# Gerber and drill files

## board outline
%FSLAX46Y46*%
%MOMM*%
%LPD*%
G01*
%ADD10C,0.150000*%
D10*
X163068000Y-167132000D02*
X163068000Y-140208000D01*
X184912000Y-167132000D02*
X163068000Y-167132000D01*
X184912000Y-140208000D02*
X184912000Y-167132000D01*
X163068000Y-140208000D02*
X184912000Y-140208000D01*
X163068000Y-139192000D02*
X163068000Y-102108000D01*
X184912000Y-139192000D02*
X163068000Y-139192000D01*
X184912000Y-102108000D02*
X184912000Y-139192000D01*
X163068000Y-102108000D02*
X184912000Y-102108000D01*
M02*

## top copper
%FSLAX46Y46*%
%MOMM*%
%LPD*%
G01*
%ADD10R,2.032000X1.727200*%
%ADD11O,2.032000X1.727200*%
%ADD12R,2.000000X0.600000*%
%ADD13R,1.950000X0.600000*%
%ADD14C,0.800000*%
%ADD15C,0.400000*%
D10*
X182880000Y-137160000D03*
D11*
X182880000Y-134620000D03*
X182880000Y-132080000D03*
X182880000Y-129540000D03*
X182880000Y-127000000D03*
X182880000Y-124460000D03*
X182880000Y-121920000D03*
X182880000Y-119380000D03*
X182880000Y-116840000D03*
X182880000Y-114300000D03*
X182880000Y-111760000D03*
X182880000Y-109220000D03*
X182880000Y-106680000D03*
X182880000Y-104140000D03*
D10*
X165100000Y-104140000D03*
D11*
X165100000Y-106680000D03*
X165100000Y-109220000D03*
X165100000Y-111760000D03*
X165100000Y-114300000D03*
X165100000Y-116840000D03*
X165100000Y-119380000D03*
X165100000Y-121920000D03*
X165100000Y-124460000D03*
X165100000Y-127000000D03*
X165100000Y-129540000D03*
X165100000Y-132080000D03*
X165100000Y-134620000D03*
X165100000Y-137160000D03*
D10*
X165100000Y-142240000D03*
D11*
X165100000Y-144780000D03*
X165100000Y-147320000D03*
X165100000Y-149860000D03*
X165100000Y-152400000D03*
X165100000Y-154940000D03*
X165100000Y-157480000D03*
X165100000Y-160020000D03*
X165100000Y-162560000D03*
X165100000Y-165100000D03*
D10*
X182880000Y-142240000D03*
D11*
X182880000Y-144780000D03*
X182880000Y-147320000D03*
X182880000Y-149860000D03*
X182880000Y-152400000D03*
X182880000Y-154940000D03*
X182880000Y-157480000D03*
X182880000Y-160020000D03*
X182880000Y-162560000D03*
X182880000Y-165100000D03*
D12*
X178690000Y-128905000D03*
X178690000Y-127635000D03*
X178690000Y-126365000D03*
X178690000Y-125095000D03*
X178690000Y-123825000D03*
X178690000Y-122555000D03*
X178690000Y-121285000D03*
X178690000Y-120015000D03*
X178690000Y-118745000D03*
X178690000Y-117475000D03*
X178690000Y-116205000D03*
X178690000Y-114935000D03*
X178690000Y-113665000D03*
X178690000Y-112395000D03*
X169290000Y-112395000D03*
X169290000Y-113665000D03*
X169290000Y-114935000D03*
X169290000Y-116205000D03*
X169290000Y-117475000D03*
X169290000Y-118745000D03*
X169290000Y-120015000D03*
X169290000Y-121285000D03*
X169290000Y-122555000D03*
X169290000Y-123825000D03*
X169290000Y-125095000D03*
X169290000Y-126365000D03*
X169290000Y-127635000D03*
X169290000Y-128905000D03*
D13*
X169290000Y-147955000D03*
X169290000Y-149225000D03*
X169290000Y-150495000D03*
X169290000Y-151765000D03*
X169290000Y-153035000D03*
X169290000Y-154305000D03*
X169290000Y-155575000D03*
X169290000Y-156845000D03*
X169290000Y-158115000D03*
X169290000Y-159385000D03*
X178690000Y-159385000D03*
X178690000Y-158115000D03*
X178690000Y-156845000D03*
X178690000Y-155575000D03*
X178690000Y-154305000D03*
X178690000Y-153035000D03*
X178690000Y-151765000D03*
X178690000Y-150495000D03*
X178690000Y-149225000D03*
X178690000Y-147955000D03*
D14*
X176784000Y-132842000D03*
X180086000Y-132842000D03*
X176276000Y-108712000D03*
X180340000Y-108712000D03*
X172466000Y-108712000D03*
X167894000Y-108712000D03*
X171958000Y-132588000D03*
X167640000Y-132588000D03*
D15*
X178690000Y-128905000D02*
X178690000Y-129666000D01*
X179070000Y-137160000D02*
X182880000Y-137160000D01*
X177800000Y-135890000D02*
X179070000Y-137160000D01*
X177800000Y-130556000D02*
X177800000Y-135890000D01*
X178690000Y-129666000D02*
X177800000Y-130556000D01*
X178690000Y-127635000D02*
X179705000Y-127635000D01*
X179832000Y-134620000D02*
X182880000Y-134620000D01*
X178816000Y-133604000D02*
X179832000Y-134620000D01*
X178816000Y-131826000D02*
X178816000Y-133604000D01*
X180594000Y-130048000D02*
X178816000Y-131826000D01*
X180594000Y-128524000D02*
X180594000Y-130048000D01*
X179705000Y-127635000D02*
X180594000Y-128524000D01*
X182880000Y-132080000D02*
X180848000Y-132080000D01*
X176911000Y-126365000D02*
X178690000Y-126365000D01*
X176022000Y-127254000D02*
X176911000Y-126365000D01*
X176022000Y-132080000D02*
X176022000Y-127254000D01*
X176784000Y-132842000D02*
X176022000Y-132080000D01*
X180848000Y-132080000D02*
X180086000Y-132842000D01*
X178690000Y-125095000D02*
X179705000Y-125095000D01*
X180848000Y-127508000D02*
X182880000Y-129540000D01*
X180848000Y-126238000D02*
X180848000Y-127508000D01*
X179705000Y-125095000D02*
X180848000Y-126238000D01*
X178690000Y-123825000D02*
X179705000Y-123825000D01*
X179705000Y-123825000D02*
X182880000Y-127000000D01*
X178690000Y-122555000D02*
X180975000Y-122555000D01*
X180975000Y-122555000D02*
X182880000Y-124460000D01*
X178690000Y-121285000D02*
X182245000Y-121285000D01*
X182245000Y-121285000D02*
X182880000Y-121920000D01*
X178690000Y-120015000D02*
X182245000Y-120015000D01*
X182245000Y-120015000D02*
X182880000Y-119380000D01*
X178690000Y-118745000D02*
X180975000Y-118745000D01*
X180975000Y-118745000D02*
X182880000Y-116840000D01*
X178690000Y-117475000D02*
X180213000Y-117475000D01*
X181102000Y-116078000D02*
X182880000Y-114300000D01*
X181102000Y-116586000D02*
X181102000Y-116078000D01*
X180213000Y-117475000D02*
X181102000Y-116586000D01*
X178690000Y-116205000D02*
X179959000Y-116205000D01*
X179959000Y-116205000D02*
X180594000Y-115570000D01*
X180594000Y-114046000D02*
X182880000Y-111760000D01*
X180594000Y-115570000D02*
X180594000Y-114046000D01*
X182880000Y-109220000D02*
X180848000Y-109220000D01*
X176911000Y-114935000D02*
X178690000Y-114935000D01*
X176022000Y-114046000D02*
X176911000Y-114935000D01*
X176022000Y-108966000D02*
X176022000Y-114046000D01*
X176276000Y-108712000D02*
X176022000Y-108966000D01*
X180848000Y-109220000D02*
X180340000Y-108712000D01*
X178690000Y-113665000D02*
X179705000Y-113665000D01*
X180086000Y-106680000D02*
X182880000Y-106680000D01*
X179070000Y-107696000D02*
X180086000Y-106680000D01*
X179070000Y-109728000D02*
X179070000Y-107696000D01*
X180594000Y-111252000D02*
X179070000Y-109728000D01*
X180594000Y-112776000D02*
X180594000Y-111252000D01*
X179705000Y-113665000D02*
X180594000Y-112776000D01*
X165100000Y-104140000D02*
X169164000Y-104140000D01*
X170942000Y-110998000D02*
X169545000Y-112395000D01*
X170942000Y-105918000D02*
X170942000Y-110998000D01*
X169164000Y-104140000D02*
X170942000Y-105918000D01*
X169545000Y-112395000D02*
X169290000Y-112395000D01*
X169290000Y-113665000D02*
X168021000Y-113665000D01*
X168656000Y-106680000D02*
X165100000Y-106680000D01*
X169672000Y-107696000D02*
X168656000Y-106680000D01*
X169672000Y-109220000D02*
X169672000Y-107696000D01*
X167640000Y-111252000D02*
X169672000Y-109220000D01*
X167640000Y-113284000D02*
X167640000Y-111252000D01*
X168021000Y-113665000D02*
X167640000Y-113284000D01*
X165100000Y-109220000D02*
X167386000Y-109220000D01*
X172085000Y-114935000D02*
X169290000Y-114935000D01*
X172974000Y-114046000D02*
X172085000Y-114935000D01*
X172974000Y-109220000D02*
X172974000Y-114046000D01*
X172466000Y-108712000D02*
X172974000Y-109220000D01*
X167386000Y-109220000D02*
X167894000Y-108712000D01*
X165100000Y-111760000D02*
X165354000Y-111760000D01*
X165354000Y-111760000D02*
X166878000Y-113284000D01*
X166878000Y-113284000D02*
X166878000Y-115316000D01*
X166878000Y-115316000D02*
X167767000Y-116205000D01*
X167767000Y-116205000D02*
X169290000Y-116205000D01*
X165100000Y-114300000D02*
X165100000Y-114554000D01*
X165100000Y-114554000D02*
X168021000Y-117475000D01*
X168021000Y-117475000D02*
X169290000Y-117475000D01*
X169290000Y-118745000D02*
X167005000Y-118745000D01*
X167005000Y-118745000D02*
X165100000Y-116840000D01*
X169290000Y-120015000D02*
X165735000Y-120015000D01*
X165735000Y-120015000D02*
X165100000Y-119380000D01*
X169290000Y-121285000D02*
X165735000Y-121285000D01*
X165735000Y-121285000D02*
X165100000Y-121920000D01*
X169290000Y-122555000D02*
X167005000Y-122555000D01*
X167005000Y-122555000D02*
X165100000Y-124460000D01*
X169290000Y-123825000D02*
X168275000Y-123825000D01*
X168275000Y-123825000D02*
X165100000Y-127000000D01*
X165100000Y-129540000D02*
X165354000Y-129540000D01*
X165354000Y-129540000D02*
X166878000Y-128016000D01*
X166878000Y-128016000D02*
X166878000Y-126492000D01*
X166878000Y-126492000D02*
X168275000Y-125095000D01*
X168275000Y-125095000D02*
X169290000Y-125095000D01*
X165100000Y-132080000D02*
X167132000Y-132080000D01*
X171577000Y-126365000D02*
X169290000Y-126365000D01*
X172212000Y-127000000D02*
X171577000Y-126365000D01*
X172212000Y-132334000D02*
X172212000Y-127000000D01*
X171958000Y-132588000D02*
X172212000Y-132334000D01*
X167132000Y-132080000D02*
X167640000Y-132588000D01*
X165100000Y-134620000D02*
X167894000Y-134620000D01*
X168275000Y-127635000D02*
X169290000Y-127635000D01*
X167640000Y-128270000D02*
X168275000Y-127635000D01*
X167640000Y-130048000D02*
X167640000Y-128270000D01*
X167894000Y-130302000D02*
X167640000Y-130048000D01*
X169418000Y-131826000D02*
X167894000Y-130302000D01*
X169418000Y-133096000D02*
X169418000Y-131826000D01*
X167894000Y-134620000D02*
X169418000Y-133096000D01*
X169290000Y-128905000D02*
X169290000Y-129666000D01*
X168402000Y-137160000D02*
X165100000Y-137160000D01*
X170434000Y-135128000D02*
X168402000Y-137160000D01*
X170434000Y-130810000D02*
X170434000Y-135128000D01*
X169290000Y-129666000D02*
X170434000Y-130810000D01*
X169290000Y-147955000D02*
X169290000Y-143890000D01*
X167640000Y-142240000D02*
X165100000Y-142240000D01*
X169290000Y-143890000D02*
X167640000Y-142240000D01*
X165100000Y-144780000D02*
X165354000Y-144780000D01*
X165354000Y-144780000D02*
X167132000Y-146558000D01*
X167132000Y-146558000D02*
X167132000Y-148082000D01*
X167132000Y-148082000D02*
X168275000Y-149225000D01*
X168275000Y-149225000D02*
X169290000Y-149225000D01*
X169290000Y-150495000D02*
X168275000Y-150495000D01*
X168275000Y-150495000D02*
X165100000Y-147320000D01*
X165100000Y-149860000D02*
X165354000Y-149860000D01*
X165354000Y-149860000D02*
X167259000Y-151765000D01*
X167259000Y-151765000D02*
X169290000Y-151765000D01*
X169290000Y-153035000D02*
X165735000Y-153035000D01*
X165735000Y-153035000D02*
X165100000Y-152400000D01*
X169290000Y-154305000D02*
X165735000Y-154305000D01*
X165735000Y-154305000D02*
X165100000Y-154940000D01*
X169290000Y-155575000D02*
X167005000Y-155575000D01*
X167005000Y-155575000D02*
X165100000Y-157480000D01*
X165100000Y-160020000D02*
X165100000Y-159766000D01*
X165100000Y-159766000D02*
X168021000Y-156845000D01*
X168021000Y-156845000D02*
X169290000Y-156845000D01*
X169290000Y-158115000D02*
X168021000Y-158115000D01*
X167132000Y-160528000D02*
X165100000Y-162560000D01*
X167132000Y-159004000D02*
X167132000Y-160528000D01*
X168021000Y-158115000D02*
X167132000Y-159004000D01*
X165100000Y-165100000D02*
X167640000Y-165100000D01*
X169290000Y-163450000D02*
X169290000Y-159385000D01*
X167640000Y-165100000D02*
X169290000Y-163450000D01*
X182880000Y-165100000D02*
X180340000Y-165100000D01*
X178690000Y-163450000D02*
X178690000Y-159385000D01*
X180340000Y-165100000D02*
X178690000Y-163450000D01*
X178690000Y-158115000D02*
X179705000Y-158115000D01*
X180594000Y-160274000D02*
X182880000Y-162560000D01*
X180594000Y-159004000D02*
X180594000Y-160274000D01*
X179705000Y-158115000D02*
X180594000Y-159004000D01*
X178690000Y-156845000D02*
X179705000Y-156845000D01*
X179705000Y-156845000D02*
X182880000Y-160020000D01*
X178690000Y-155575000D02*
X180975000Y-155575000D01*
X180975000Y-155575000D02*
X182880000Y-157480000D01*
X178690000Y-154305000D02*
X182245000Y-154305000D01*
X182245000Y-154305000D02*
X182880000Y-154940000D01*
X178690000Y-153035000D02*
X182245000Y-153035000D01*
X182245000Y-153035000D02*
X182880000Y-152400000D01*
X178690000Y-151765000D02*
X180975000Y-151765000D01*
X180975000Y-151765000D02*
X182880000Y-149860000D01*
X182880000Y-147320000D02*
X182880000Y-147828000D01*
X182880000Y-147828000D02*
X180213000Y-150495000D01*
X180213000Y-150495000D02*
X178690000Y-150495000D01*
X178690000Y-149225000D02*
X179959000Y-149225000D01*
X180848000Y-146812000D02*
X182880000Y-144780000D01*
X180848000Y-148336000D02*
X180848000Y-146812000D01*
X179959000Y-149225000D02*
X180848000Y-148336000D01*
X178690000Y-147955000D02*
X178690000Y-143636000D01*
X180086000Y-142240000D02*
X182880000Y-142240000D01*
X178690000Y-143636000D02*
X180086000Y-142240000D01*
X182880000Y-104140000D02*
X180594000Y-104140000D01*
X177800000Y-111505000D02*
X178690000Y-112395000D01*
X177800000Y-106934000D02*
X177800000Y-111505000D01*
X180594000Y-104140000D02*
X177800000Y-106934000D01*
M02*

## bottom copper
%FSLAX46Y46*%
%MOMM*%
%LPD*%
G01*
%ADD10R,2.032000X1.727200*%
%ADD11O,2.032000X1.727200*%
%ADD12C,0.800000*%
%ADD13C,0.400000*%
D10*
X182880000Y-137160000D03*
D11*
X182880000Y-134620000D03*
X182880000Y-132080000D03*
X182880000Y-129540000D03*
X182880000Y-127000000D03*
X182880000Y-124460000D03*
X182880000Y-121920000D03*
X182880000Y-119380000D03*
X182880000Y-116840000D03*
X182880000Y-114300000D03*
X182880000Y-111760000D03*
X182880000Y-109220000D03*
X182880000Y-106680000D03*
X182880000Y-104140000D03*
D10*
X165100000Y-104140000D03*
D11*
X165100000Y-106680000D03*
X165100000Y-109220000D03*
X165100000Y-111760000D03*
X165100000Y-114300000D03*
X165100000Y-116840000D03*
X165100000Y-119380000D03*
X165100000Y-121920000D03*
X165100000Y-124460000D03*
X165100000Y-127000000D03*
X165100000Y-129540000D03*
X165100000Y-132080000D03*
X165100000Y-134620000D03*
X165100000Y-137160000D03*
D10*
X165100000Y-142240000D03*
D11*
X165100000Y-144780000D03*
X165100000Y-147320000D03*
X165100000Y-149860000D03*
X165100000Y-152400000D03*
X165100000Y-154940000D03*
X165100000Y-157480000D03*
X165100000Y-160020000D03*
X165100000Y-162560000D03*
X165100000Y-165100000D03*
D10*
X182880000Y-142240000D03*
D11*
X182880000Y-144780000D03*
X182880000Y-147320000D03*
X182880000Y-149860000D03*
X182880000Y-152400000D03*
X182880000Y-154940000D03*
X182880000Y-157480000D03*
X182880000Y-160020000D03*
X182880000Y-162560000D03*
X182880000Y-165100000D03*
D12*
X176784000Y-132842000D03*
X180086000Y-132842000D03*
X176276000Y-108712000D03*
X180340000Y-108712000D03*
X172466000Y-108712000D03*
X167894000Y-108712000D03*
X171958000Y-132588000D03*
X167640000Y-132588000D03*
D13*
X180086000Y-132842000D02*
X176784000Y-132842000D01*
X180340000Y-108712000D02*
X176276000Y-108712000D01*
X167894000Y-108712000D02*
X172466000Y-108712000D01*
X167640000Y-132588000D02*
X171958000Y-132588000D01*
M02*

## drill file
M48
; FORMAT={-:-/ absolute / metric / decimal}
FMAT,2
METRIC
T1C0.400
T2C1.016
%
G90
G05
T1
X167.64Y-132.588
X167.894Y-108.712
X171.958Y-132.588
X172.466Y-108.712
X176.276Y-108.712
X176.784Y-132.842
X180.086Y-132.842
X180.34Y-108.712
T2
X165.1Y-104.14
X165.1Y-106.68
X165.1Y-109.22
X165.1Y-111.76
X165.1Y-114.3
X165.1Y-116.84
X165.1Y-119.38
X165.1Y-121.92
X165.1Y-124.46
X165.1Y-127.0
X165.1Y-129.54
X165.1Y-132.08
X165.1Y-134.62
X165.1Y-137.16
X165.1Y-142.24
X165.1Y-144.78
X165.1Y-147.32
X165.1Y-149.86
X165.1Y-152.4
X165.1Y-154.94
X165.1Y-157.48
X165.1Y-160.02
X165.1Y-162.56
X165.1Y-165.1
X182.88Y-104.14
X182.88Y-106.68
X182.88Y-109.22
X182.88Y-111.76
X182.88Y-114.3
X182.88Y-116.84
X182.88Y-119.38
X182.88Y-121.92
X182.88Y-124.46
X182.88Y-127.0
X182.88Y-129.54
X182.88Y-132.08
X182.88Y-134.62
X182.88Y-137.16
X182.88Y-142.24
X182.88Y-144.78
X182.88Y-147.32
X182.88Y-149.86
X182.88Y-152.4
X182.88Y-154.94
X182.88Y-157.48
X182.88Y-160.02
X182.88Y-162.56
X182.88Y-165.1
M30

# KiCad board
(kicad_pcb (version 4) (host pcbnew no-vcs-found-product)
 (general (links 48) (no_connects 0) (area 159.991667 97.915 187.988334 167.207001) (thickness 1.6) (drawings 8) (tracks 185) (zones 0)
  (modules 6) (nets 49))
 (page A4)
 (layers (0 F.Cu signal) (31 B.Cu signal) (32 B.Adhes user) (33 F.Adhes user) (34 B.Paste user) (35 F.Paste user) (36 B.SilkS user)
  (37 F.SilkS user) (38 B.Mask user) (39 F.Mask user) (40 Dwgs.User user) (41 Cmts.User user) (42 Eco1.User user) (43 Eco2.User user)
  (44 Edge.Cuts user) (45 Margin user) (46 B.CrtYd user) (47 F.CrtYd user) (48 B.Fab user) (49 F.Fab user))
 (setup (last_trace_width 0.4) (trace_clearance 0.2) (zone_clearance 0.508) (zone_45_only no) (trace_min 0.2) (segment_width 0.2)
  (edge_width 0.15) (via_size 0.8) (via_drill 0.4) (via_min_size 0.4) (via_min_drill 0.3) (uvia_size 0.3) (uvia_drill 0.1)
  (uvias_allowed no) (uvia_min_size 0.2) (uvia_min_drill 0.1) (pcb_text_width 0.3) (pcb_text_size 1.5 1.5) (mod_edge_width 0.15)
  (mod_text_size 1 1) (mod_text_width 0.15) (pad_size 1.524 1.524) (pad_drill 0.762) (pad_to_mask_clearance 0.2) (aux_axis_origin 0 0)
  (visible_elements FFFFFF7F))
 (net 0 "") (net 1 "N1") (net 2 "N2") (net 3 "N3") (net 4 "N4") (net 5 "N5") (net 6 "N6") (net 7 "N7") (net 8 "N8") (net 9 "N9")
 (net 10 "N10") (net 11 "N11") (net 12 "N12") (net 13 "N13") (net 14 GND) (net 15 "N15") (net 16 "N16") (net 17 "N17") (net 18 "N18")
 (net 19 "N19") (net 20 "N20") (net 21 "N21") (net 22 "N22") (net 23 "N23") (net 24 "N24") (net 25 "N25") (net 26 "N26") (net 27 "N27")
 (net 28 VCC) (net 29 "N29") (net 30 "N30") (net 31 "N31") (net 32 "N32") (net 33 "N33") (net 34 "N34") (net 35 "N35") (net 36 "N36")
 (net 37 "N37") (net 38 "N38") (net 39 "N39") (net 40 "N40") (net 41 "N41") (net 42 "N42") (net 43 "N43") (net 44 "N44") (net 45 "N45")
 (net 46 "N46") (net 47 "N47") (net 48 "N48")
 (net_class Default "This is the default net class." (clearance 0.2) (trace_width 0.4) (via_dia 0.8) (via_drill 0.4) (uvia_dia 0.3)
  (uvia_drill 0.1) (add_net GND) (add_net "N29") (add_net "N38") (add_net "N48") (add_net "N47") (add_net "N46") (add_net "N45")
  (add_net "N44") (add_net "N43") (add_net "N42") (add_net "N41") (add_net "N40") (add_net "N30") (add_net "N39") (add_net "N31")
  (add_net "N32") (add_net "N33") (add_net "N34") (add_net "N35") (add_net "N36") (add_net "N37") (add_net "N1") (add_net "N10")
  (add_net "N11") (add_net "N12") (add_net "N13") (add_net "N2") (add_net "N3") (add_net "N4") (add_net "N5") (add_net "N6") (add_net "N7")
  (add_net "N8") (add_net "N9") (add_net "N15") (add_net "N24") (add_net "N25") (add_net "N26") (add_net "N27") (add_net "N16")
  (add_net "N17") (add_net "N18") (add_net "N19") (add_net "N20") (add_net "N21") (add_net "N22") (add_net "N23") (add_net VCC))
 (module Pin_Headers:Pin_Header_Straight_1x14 (layer F.Cu) (at 182.88 137.16 180)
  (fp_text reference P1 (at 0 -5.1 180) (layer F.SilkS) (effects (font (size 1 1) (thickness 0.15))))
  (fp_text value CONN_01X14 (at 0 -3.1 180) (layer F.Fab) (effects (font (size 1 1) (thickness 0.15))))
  (pad 1 thru_hole rect (at 0 0 180) (size 2.032 1.7272) (drill 1.016) (layers *.Cu *.Mask F.SilkS) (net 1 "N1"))
  (pad 2 thru_hole oval (at 0 2.54 180) (size 2.032 1.7272) (drill 1.016) (layers *.Cu *.Mask F.SilkS) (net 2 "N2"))
  (pad 3 thru_hole oval (at 0 5.08 180) (size 2.032 1.7272) (drill 1.016) (layers *.Cu *.Mask F.SilkS) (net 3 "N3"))
  (pad 4 thru_hole oval (at 0 7.62 180) (size 2.032 1.7272) (drill 1.016) (layers *.Cu *.Mask F.SilkS) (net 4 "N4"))
  (pad 5 thru_hole oval (at 0 10.16 180) (size 2.032 1.7272) (drill 1.016) (layers *.Cu *.Mask F.SilkS) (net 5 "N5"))
  (pad 6 thru_hole oval (at 0 12.7 180) (size 2.032 1.7272) (drill 1.016) (layers *.Cu *.Mask F.SilkS) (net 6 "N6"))
  (pad 7 thru_hole oval (at 0 15.24 180) (size 2.032 1.7272) (drill 1.016) (layers *.Cu *.Mask F.SilkS) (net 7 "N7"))
  (pad 8 thru_hole oval (at 0 17.78 180) (size 2.032 1.7272) (drill 1.016) (layers *.Cu *.Mask F.SilkS) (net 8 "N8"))
  (pad 9 thru_hole oval (at 0 20.32 180) (size 2.032 1.7272) (drill 1.016) (layers *.Cu *.Mask F.SilkS) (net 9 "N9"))
  (pad 10 thru_hole oval (at 0 22.86 180) (size 2.032 1.7272) (drill 1.016) (layers *.Cu *.Mask F.SilkS) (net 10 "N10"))
  (pad 11 thru_hole oval (at 0 25.4 180) (size 2.032 1.7272) (drill 1.016) (layers *.Cu *.Mask F.SilkS) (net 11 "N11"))
  (pad 12 thru_hole oval (at 0 27.94 180) (size 2.032 1.7272) (drill 1.016) (layers *.Cu *.Mask F.SilkS) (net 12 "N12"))
  (pad 13 thru_hole oval (at 0 30.48 180) (size 2.032 1.7272) (drill 1.016) (layers *.Cu *.Mask F.SilkS) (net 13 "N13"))
  (pad 14 thru_hole oval (at 0 33.02 180) (size 2.032 1.7272) (drill 1.016) (layers *.Cu *.Mask F.SilkS) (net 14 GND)))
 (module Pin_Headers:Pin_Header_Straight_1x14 (layer F.Cu) (at 165.1 104.14)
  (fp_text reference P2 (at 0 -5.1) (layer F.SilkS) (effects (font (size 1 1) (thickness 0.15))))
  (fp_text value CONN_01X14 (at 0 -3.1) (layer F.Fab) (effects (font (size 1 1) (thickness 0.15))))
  (pad 1 thru_hole rect (at 0 0) (size 2.032 1.7272) (drill 1.016) (layers *.Cu *.Mask F.SilkS) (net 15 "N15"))
  (pad 2 thru_hole oval (at 0 2.54) (size 2.032 1.7272) (drill 1.016) (layers *.Cu *.Mask F.SilkS) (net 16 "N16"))
  (pad 3 thru_hole oval (at 0 5.08) (size 2.032 1.7272) (drill 1.016) (layers *.Cu *.Mask F.SilkS) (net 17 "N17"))
  (pad 4 thru_hole oval (at 0 7.62) (size 2.032 1.7272) (drill 1.016) (layers *.Cu *.Mask F.SilkS) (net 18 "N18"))
  (pad 5 thru_hole oval (at 0 10.16) (size 2.032 1.7272) (drill 1.016) (layers *.Cu *.Mask F.SilkS) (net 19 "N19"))
  (pad 6 thru_hole oval (at 0 12.7) (size 2.032 1.7272) (drill 1.016) (layers *.Cu *.Mask F.SilkS) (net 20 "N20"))
  (pad 7 thru_hole oval (at 0 15.24) (size 2.032 1.7272) (drill 1.016) (layers *.Cu *.Mask F.SilkS) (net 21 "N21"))
  (pad 8 thru_hole oval (at 0 17.78) (size 2.032 1.7272) (drill 1.016) (layers *.Cu *.Mask F.SilkS) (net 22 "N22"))
  (pad 9 thru_hole oval (at 0 20.32) (size 2.032 1.7272) (drill 1.016) (layers *.Cu *.Mask F.SilkS) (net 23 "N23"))
  (pad 10 thru_hole oval (at 0 22.86) (size 2.032 1.7272) (drill 1.016) (layers *.Cu *.Mask F.SilkS) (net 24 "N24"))
  (pad 11 thru_hole oval (at 0 25.4) (size 2.032 1.7272) (drill 1.016) (layers *.Cu *.Mask F.SilkS) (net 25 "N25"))
  (pad 12 thru_hole oval (at 0 27.94) (size 2.032 1.7272) (drill 1.016) (layers *.Cu *.Mask F.SilkS) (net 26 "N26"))
  (pad 13 thru_hole oval (at 0 30.48) (size 2.032 1.7272) (drill 1.016) (layers *.Cu *.Mask F.SilkS) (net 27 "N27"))
  (pad 14 thru_hole oval (at 0 33.02) (size 2.032 1.7272) (drill 1.016) (layers *.Cu *.Mask F.SilkS) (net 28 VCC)))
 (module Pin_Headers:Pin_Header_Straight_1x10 (layer F.Cu) (at 165.1 142.24)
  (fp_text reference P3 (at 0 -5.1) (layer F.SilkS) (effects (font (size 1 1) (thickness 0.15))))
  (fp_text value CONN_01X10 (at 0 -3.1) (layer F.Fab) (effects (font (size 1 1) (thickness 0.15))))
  (pad 1 thru_hole rect (at 0 0) (size 2.032 1.7272) (drill 1.016) (layers *.Cu *.Mask F.SilkS) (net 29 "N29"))
  (pad 2 thru_hole oval (at 0 2.54) (size 2.032 1.7272) (drill 1.016) (layers *.Cu *.Mask F.SilkS) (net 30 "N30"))
  (pad 3 thru_hole oval (at 0 5.08) (size 2.032 1.7272) (drill 1.016) (layers *.Cu *.Mask F.SilkS) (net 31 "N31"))
  (pad 4 thru_hole oval (at 0 7.62) (size 2.032 1.7272) (drill 1.016) (layers *.Cu *.Mask F.SilkS) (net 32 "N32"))
  (pad 5 thru_hole oval (at 0 10.16) (size 2.032 1.7272) (drill 1.016) (layers *.Cu *.Mask F.SilkS) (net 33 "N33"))
  (pad 6 thru_hole oval (at 0 12.7) (size 2.032 1.7272) (drill 1.016) (layers *.Cu *.Mask F.SilkS) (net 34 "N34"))
  (pad 7 thru_hole oval (at 0 15.24) (size 2.032 1.7272) (drill 1.016) (layers *.Cu *.Mask F.SilkS) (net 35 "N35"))
  (pad 8 thru_hole oval (at 0 17.78) (size 2.032 1.7272) (drill 1.016) (layers *.Cu *.Mask F.SilkS) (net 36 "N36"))
  (pad 9 thru_hole oval (at 0 20.32) (size 2.032 1.7272) (drill 1.016) (layers *.Cu *.Mask F.SilkS) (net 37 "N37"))
  (pad 10 thru_hole oval (at 0 22.86) (size 2.032 1.7272) (drill 1.016) (layers *.Cu *.Mask F.SilkS) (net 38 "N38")))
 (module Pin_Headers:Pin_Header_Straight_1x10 (layer F.Cu) (at 182.88 142.24)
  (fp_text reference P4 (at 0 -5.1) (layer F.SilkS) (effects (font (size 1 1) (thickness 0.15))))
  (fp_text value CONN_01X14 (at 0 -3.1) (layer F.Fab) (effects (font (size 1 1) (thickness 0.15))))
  (pad 1 thru_hole rect (at 0 0) (size 2.032 1.7272) (drill 1.016) (layers *.Cu *.Mask F.SilkS) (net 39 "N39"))
  (pad 2 thru_hole oval (at 0 2.54) (size 2.032 1.7272) (drill 1.016) (layers *.Cu *.Mask F.SilkS) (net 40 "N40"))
  (pad 3 thru_hole oval (at 0 5.08) (size 2.032 1.7272) (drill 1.016) (layers *.Cu *.Mask F.SilkS) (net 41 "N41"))
  (pad 4 thru_hole oval (at 0 7.62) (size 2.032 1.7272) (drill 1.016) (layers *.Cu *.Mask F.SilkS) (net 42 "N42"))
  (pad 5 thru_hole oval (at 0 10.16) (size 2.032 1.7272) (drill 1.016) (layers *.Cu *.Mask F.SilkS) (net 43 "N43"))
  (pad 6 thru_hole oval (at 0 12.7) (size 2.032 1.7272) (drill 1.016) (layers *.Cu *.Mask F.SilkS) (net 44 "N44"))
  (pad 7 thru_hole oval (at 0 15.24) (size 2.032 1.7272) (drill 1.016) (layers *.Cu *.Mask F.SilkS) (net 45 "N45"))
  (pad 8 thru_hole oval (at 0 17.78) (size 2.032 1.7272) (drill 1.016) (layers *.Cu *.Mask F.SilkS) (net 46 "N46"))
  (pad 9 thru_hole oval (at 0 20.32) (size 2.032 1.7272) (drill 1.016) (layers *.Cu *.Mask F.SilkS) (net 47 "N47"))
  (pad 10 thru_hole oval (at 0 22.86) (size 2.032 1.7272) (drill 1.016) (layers *.Cu *.Mask F.SilkS) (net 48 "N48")))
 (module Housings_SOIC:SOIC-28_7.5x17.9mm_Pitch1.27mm (layer F.Cu) (at 173.99 120.65 180)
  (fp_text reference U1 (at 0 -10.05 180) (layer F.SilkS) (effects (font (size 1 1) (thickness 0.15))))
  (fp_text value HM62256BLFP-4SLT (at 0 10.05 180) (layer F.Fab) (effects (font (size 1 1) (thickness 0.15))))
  (pad 1 smd rect (at -4.7 -8.255 180) (size 2 0.6) (layers F.Cu F.Paste F.Mask) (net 1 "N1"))
  (pad 2 smd rect (at -4.7 -6.985 180) (size 2 0.6) (layers F.Cu F.Paste F.Mask) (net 2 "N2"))
  (pad 3 smd rect (at -4.7 -5.715 180) (size 2 0.6) (layers F.Cu F.Paste F.Mask) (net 3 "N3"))
  (pad 4 smd rect (at -4.7 -4.445 180) (size 2 0.6) (layers F.Cu F.Paste F.Mask) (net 4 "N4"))
  (pad 5 smd rect (at -4.7 -3.175 180) (size 2 0.6) (layers F.Cu F.Paste F.Mask) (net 5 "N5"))
  (pad 6 smd rect (at -4.7 -1.905 180) (size 2 0.6) (layers F.Cu F.Paste F.Mask) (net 6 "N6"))
  (pad 7 smd rect (at -4.7 -0.635 180) (size 2 0.6) (layers F.Cu F.Paste F.Mask) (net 7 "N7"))
  (pad 8 smd rect (at -4.7 0.635 180) (size 2 0.6) (layers F.Cu F.Paste F.Mask) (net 8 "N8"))
  (pad 9 smd rect (at -4.7 1.905 180) (size 2 0.6) (layers F.Cu F.Paste F.Mask) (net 9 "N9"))
  (pad 10 smd rect (at -4.7 3.175 180) (size 2 0.6) (layers F.Cu F.Paste F.Mask) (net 10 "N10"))
  (pad 11 smd rect (at -4.7 4.445 180) (size 2 0.6) (layers F.Cu F.Paste F.Mask) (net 11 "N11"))
  (pad 12 smd rect (at -4.7 5.715 180) (size 2 0.6) (layers F.Cu F.Paste F.Mask) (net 12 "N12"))
  (pad 13 smd rect (at -4.7 6.985 180) (size 2 0.6) (layers F.Cu F.Paste F.Mask) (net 13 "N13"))
  (pad 14 smd rect (at -4.7 8.255 180) (size 2 0.6) (layers F.Cu F.Paste F.Mask) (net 14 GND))
  (pad 15 smd rect (at 4.7 8.255 180) (size 2 0.6) (layers F.Cu F.Paste F.Mask) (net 15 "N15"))
  (pad 16 smd rect (at 4.7 6.985 180) (size 2 0.6) (layers F.Cu F.Paste F.Mask) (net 16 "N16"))
  (pad 17 smd rect (at 4.7 5.715 180) (size 2 0.6) (layers F.Cu F.Paste F.Mask) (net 17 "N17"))
  (pad 18 smd rect (at 4.7 4.445 180) (size 2 0.6) (layers F.Cu F.Paste F.Mask) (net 18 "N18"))
  (pad 19 smd rect (at 4.7 3.175 180) (size 2 0.6) (layers F.Cu F.Paste F.Mask) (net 19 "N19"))
  (pad 20 smd rect (at 4.7 1.905 180) (size 2 0.6) (layers F.Cu F.Paste F.Mask) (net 20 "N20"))
  (pad 21 smd rect (at 4.7 0.635 180) (size 2 0.6) (layers F.Cu F.Paste F.Mask) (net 21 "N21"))
  (pad 22 smd rect (at 4.7 -0.635 180) (size 2 0.6) (layers F.Cu F.Paste F.Mask) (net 22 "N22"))
  (pad 23 smd rect (at 4.7 -1.905 180) (size 2 0.6) (layers F.Cu F.Paste F.Mask) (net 23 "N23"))
  (pad 24 smd rect (at 4.7 -3.175 180) (size 2 0.6) (layers F.Cu F.Paste F.Mask) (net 24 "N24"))
  (pad 25 smd rect (at 4.7 -4.445 180) (size 2 0.6) (layers F.Cu F.Paste F.Mask) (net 25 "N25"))
  (pad 26 smd rect (at 4.7 -5.715 180) (size 2 0.6) (layers F.Cu F.Paste F.Mask) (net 26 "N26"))
  (pad 27 smd rect (at 4.7 -6.985 180) (size 2 0.6) (layers F.Cu F.Paste F.Mask) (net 27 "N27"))
  (pad 28 smd rect (at 4.7 -8.255 180) (size 2 0.6) (layers F.Cu F.Paste F.Mask) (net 28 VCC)))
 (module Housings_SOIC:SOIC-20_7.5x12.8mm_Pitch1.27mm (layer F.Cu) (at 173.99 153.67)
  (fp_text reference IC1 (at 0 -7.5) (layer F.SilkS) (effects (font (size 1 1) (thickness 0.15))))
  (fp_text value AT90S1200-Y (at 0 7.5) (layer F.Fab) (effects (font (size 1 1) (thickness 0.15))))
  (pad 1 smd rect (at -4.7 -5.715) (size 1.95 0.6) (layers F.Cu F.Paste F.Mask) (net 29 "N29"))
  (pad 2 smd rect (at -4.7 -4.445) (size 1.95 0.6) (layers F.Cu F.Paste F.Mask) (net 30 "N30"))
  (pad 3 smd rect (at -4.7 -3.175) (size 1.95 0.6) (layers F.Cu F.Paste F.Mask) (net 31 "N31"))
  (pad 4 smd rect (at -4.7 -1.905) (size 1.95 0.6) (layers F.Cu F.Paste F.Mask) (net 32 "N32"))
  (pad 5 smd rect (at -4.7 -0.635) (size 1.95 0.6) (layers F.Cu F.Paste F.Mask) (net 33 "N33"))
  (pad 6 smd rect (at -4.7 0.635) (size 1.95 0.6) (layers F.Cu F.Paste F.Mask) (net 34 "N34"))
  (pad 7 smd rect (at -4.7 1.905) (size 1.95 0.6) (layers F.Cu F.Paste F.Mask) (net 35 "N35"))
  (pad 8 smd rect (at -4.7 3.175) (size 1.95 0.6) (layers F.Cu F.Paste F.Mask) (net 36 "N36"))
  (pad 9 smd rect (at -4.7 4.445) (size 1.95 0.6) (layers F.Cu F.Paste F.Mask) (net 37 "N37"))
  (pad 10 smd rect (at -4.7 5.715) (size 1.95 0.6) (layers F.Cu F.Paste F.Mask) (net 38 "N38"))
  (pad 11 smd rect (at 4.7 5.715) (size 1.95 0.6) (layers F.Cu F.Paste F.Mask) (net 48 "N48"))
  (pad 12 smd rect (at 4.7 4.445) (size 1.95 0.6) (layers F.Cu F.Paste F.Mask) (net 47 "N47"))
  (pad 13 smd rect (at 4.7 3.175) (size 1.95 0.6) (layers F.Cu F.Paste F.Mask) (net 46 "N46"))
  (pad 14 smd rect (at 4.7 1.905) (size 1.95 0.6) (layers F.Cu F.Paste F.Mask) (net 45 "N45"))
  (pad 15 smd rect (at 4.7 0.635) (size 1.95 0.6) (layers F.Cu F.Paste F.Mask) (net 44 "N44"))
  (pad 16 smd rect (at 4.7 -0.635) (size 1.95 0.6) (layers F.Cu F.Paste F.Mask) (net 43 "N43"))
  (pad 17 smd rect (at 4.7 -1.905) (size 1.95 0.6) (layers F.Cu F.Paste F.Mask) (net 42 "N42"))
  (pad 18 smd rect (at 4.7 -3.175) (size 1.95 0.6) (layers F.Cu F.Paste F.Mask) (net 41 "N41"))
  (pad 19 smd rect (at 4.7 -4.445) (size 1.95 0.6) (layers F.Cu F.Paste F.Mask) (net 40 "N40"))
  (pad 20 smd rect (at 4.7 -5.715) (size 1.95 0.6) (layers F.Cu F.Paste F.Mask) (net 39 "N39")))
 (gr_line (start 163.068 167.132) (end 163.068 140.208) (angle 90) (layer Edge.Cuts) (width 0.15))
 (gr_line (start 184.912 167.132) (end 163.068 167.132) (angle 90) (layer Edge.Cuts) (width 0.15))
 (gr_line (start 184.912 140.208) (end 184.912 167.132) (angle 90) (layer Edge.Cuts) (width 0.15))
 (gr_line (start 163.068 140.208) (end 184.912 140.208) (angle 90) (layer Edge.Cuts) (width 0.15))
 (gr_line (start 163.068 139.192) (end 163.068 102.108) (angle 90) (layer Edge.Cuts) (width 0.15))
 (gr_line (start 184.912 139.192) (end 163.068 139.192) (angle 90) (layer Edge.Cuts) (width 0.15))
 (gr_line (start 184.912 102.108) (end 184.912 139.192) (angle 90) (layer Edge.Cuts) (width 0.15))
 (gr_line (start 163.068 102.108) (end 184.912 102.108) (angle 90) (layer Edge.Cuts) (width 0.15))
 (segment (start 178.69 128.905) (end 178.69 129.666) (width 0.4) (layer F.Cu) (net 1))
 (segment (start 179.07 137.16) (end 182.88 137.16) (width 0.4) (layer F.Cu) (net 1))
 (segment (start 177.8 135.89) (end 179.07 137.16) (width 0.4) (layer F.Cu) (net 1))
 (segment (start 177.8 130.556) (end 177.8 135.89) (width 0.4) (layer F.Cu) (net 1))
 (segment (start 178.69 129.666) (end 177.8 130.556) (width 0.4) (layer F.Cu) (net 1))
 (segment (start 178.69 127.635) (end 179.705 127.635) (width 0.4) (layer F.Cu) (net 2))
 (segment (start 179.832 134.62) (end 182.88 134.62) (width 0.4) (layer F.Cu) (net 2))
 (segment (start 178.816 133.604) (end 179.832 134.62) (width 0.4) (layer F.Cu) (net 2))
 (segment (start 178.816 131.826) (end 178.816 133.604) (width 0.4) (layer F.Cu) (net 2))
 (segment (start 180.594 130.048) (end 178.816 131.826) (width 0.4) (layer F.Cu) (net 2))
 (segment (start 180.594 128.524) (end 180.594 130.048) (width 0.4) (layer F.Cu) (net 2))
 (segment (start 179.705 127.635) (end 180.594 128.524) (width 0.4) (layer F.Cu) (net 2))
 (segment (start 182.88 132.08) (end 180.848 132.08) (width 0.4) (layer F.Cu) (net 3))
 (segment (start 176.911 126.365) (end 178.69 126.365) (width 0.4) (layer F.Cu) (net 3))
 (segment (start 176.022 127.254) (end 176.911 126.365) (width 0.4) (layer F.Cu) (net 3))
 (segment (start 176.022 132.08) (end 176.022 127.254) (width 0.4) (layer F.Cu) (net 3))
 (segment (start 176.784 132.842) (end 176.022 132.08) (width 0.4) (layer F.Cu) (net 3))
 (via (at 176.784 132.842) (size 0.8) (drill 0.4) (layers F.Cu B.Cu) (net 3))
 (segment (start 180.086 132.842) (end 176.784 132.842) (width 0.4) (layer B.Cu) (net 3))
 (via (at 180.086 132.842) (size 0.8) (drill 0.4) (layers F.Cu B.Cu) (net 3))
 (segment (start 180.848 132.08) (end 180.086 132.842) (width 0.4) (layer F.Cu) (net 3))
 (segment (start 178.69 125.095) (end 179.705 125.095) (width 0.4) (layer F.Cu) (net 4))
 (segment (start 180.848 127.508) (end 182.88 129.54) (width 0.4) (layer F.Cu) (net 4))
 (segment (start 180.848 126.238) (end 180.848 127.508) (width 0.4) (layer F.Cu) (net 4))
 (segment (start 179.705 125.095) (end 180.848 126.238) (width 0.4) (layer F.Cu) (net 4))
 (segment (start 178.69 123.825) (end 179.705 123.825) (width 0.4) (layer F.Cu) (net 5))
 (segment (start 179.705 123.825) (end 182.88 127) (width 0.4) (layer F.Cu) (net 5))
 (segment (start 178.69 122.555) (end 180.975 122.555) (width 0.4) (layer F.Cu) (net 6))
 (segment (start 180.975 122.555) (end 182.88 124.46) (width 0.4) (layer F.Cu) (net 6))
 (segment (start 178.69 121.285) (end 182.245 121.285) (width 0.4) (layer F.Cu) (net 7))
 (segment (start 182.245 121.285) (end 182.88 121.92) (width 0.4) (layer F.Cu) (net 7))
 (segment (start 178.69 120.015) (end 182.245 120.015) (width 0.4) (layer F.Cu) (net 8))
 (segment (start 182.245 120.015) (end 182.88 119.38) (width 0.4) (layer F.Cu) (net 8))
 (segment (start 178.69 118.745) (end 180.975 118.745) (width 0.4) (layer F.Cu) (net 9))
 (segment (start 180.975 118.745) (end 182.88 116.84) (width 0.4) (layer F.Cu) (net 9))
 (segment (start 178.69 117.475) (end 180.213 117.475) (width 0.4) (layer F.Cu) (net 10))
 (segment (start 181.102 116.078) (end 182.88 114.3) (width 0.4) (layer F.Cu) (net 10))
 (segment (start 181.102 116.586) (end 181.102 116.078) (width 0.4) (layer F.Cu) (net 10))
 (segment (start 180.213 117.475) (end 181.102 116.586) (width 0.4) (layer F.Cu) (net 10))
 (segment (start 178.69 116.205) (end 179.959 116.205) (width 0.4) (layer F.Cu) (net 11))
 (segment (start 179.959 116.205) (end 180.594 115.57) (width 0.4) (layer F.Cu) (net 11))
 (segment (start 180.594 114.046) (end 182.88 111.76) (width 0.4) (layer F.Cu) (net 11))
 (segment (start 180.594 115.57) (end 180.594 114.046) (width 0.4) (layer F.Cu) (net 11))
 (segment (start 182.88 109.22) (end 180.848 109.22) (width 0.4) (layer F.Cu) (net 12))
 (segment (start 176.911 114.935) (end 178.69 114.935) (width 0.4) (layer F.Cu) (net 12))
 (segment (start 176.022 114.046) (end 176.911 114.935) (width 0.4) (layer F.Cu) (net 12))
 (segment (start 176.022 108.966) (end 176.022 114.046) (width 0.4) (layer F.Cu) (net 12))
 (segment (start 176.276 108.712) (end 176.022 108.966) (width 0.4) (layer F.Cu) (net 12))
 (via (at 176.276 108.712) (size 0.8) (drill 0.4) (layers F.Cu B.Cu) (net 12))
 (segment (start 180.34 108.712) (end 176.276 108.712) (width 0.4) (layer B.Cu) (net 12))
 (via (at 180.34 108.712) (size 0.8) (drill 0.4) (layers F.Cu B.Cu) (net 12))
 (segment (start 180.848 109.22) (end 180.34 108.712) (width 0.4) (layer F.Cu) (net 12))
 (segment (start 178.69 113.665) (end 179.705 113.665) (width 0.4) (layer F.Cu) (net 13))
 (segment (start 180.086 106.68) (end 182.88 106.68) (width 0.4) (layer F.Cu) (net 13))
 (segment (start 179.07 107.696) (end 180.086 106.68) (width 0.4) (layer F.Cu) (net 13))
 (segment (start 179.07 109.728) (end 179.07 107.696) (width 0.4) (layer F.Cu) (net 13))
 (segment (start 180.594 111.252) (end 179.07 109.728) (width 0.4) (layer F.Cu) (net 13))
 (segment (start 180.594 112.776) (end 180.594 111.252) (width 0.4) (layer F.Cu) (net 13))
 (segment (start 179.705 113.665) (end 180.594 112.776) (width 0.4) (layer F.Cu) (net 13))
 (segment (start 165.1 104.14) (end 169.164 104.14) (width 0.4) (layer F.Cu) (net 15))
 (segment (start 170.942 110.998) (end 169.545 112.395) (width 0.4) (layer F.Cu) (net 15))
 (segment (start 170.942 105.918) (end 170.942 110.998) (width 0.4) (layer F.Cu) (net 15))
 (segment (start 169.164 104.14) (end 170.942 105.918) (width 0.4) (layer F.Cu) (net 15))
 (segment (start 169.545 112.395) (end 169.29 112.395) (width 0.4) (layer F.Cu) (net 15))
 (segment (start 169.29 113.665) (end 168.021 113.665) (width 0.4) (layer F.Cu) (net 16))
 (segment (start 168.656 106.68) (end 165.1 106.68) (width 0.4) (layer F.Cu) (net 16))
 (segment (start 169.672 107.696) (end 168.656 106.68) (width 0.4) (layer F.Cu) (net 16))
 (segment (start 169.672 109.22) (end 169.672 107.696) (width 0.4) (layer F.Cu) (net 16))
 (segment (start 167.64 111.252) (end 169.672 109.22) (width 0.4) (layer F.Cu) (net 16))
 (segment (start 167.64 113.284) (end 167.64 111.252) (width 0.4) (layer F.Cu) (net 16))
 (segment (start 168.021 113.665) (end 167.64 113.284) (width 0.4) (layer F.Cu) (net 16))
 (segment (start 165.1 109.22) (end 167.386 109.22) (width 0.4) (layer F.Cu) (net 17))
 (segment (start 172.085 114.935) (end 169.29 114.935) (width 0.4) (layer F.Cu) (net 17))
 (segment (start 172.974 114.046) (end 172.085 114.935) (width 0.4) (layer F.Cu) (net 17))
 (segment (start 172.974 109.22) (end 172.974 114.046) (width 0.4) (layer F.Cu) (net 17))
 (segment (start 172.466 108.712) (end 172.974 109.22) (width 0.4) (layer F.Cu) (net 17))
 (via (at 172.466 108.712) (size 0.8) (drill 0.4) (layers F.Cu B.Cu) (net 17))
 (segment (start 167.894 108.712) (end 172.466 108.712) (width 0.4) (layer B.Cu) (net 17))
 (via (at 167.894 108.712) (size 0.8) (drill 0.4) (layers F.Cu B.Cu) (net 17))
 (segment (start 167.386 109.22) (end 167.894 108.712) (width 0.4) (layer F.Cu) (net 17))
 (segment (start 165.1 111.76) (end 165.354 111.76) (width 0.4) (layer F.Cu) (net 18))
 (segment (start 165.354 111.76) (end 166.878 113.284) (width 0.4) (layer F.Cu) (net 18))
 (segment (start 166.878 113.284) (end 166.878 115.316) (width 0.4) (layer F.Cu) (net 18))
 (segment (start 166.878 115.316) (end 167.767 116.205) (width 0.4) (layer F.Cu) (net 18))
 (segment (start 167.767 116.205) (end 169.29 116.205) (width 0.4) (layer F.Cu) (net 18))
 (segment (start 165.1 114.3) (end 165.1 114.554) (width 0.4) (layer F.Cu) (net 19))
 (segment (start 165.1 114.554) (end 168.021 117.475) (width 0.4) (layer F.Cu) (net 19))
 (segment (start 168.021 117.475) (end 169.29 117.475) (width 0.4) (layer F.Cu) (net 19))
 (segment (start 169.29 118.745) (end 167.005 118.745) (width 0.4) (layer F.Cu) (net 20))
 (segment (start 167.005 118.745) (end 165.1 116.84) (width 0.4) (layer F.Cu) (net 20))
 (segment (start 169.29 120.015) (end 165.735 120.015) (width 0.4) (layer F.Cu) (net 21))
 (segment (start 165.735 120.015) (end 165.1 119.38) (width 0.4) (layer F.Cu) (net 21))
 (segment (start 169.29 121.285) (end 165.735 121.285) (width 0.4) (layer F.Cu) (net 22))
 (segment (start 165.735 121.285) (end 165.1 121.92) (width 0.4) (layer F.Cu) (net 22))
 (segment (start 169.29 122.555) (end 167.005 122.555) (width 0.4) (layer F.Cu) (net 23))
 (segment (start 167.005 122.555) (end 165.1 124.46) (width 0.4) (layer F.Cu) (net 23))
 (segment (start 169.29 123.825) (end 168.275 123.825) (width 0.4) (layer F.Cu) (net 24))
 (segment (start 168.275 123.825) (end 165.1 127) (width 0.4) (layer F.Cu) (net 24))
 (segment (start 165.1 129.54) (end 165.354 129.54) (width 0.4) (layer F.Cu) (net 25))
 (segment (start 165.354 129.54) (end 166.878 128.016) (width 0.4) (layer F.Cu) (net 25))
 (segment (start 166.878 128.016) (end 166.878 126.492) (width 0.4) (layer F.Cu) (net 25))
 (segment (start 166.878 126.492) (end 168.275 125.095) (width 0.4) (layer F.Cu) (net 25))
 (segment (start 168.275 125.095) (end 169.29 125.095) (width 0.4) (layer F.Cu) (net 25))
 (segment (start 165.1 132.08) (end 167.132 132.08) (width 0.4) (layer F.Cu) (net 26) (status 400000))
 (segment (start 171.577 126.365) (end 169.29 126.365) (width 0.4) (layer F.Cu) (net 26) (status 800000))
 (segment (start 172.212 127) (end 171.577 126.365) (width 0.4) (layer F.Cu) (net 26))
 (segment (start 172.212 132.334) (end 172.212 127) (width 0.4) (layer F.Cu) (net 26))
 (segment (start 171.958 132.588) (end 172.212 132.334) (width 0.4) (layer F.Cu) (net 26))
 (via (at 171.958 132.588) (size 0.8) (drill 0.4) (layers F.Cu B.Cu) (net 26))
 (segment (start 167.64 132.588) (end 171.958 132.588) (width 0.4) (layer B.Cu) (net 26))
 (via (at 167.64 132.588) (size 0.8) (drill 0.4) (layers F.Cu B.Cu) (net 26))
 (segment (start 167.132 132.08) (end 167.64 132.588) (width 0.4) (layer F.Cu) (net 26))
 (segment (start 165.1 134.62) (end 167.894 134.62) (width 0.4) (layer F.Cu) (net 27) (status 400000))
 (segment (start 168.275 127.635) (end 169.29 127.635) (width 0.4) (layer F.Cu) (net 27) (status 800000))
 (segment (start 167.64 128.27) (end 168.275 127.635) (width 0.4) (layer F.Cu) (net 27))
 (segment (start 167.64 130.048) (end 167.64 128.27) (width 0.4) (layer F.Cu) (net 27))
 (segment (start 167.894 130.302) (end 167.64 130.048) (width 0.4) (layer F.Cu) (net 27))
 (segment (start 169.418 131.826) (end 167.894 130.302) (width 0.4) (layer F.Cu) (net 27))
 (segment (start 169.418 133.096) (end 169.418 131.826) (width 0.4) (layer F.Cu) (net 27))
 (segment (start 167.894 134.62) (end 169.418 133.096) (width 0.4) (layer F.Cu) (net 27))
 (segment (start 169.29 128.905) (end 169.29 129.666) (width 0.4) (layer F.Cu) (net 28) (status 400000))
 (segment (start 168.402 137.16) (end 165.1 137.16) (width 0.4) (layer F.Cu) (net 28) (status 800000))
 (segment (start 170.434 135.128) (end 168.402 137.16) (width 0.4) (layer F.Cu) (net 28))
 (segment (start 170.434 130.81) (end 170.434 135.128) (width 0.4) (layer F.Cu) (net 28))
 (segment (start 169.29 129.666) (end 170.434 130.81) (width 0.4) (layer F.Cu) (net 28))
 (segment (start 169.29 147.955) (end 169.29 143.89) (width 0.4) (layer F.Cu) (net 29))
 (segment (start 167.64 142.24) (end 165.1 142.24) (width 0.4) (layer F.Cu) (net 29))
 (segment (start 169.29 143.89) (end 167.64 142.24) (width 0.4) (layer F.Cu) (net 29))
 (segment (start 165.1 144.78) (end 165.354 144.78) (width 0.4) (layer F.Cu) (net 30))
 (segment (start 165.354 144.78) (end 167.132 146.558) (width 0.4) (layer F.Cu) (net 30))
 (segment (start 167.132 146.558) (end 167.132 148.082) (width 0.4) (layer F.Cu) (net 30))
 (segment (start 167.132 148.082) (end 168.275 149.225) (width 0.4) (layer F.Cu) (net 30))
 (segment (start 168.275 149.225) (end 169.29 149.225) (width 0.4) (layer F.Cu) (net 30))
 (segment (start 169.29 150.495) (end 168.275 150.495) (width 0.4) (layer F.Cu) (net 31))
 (segment (start 168.275 150.495) (end 165.1 147.32) (width 0.4) (layer F.Cu) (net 31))
 (segment (start 165.1 149.86) (end 165.354 149.86) (width 0.4) (layer F.Cu) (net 32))
 (segment (start 165.354 149.86) (end 167.259 151.765) (width 0.4) (layer F.Cu) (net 32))
 (segment (start 167.259 151.765) (end 169.29 151.765) (width 0.4) (layer F.Cu) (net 32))
 (segment (start 169.29 153.035) (end 165.735 153.035) (width 0.4) (layer F.Cu) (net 33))
 (segment (start 165.735 153.035) (end 165.1 152.4) (width 0.4) (layer F.Cu) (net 33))
 (segment (start 169.29 154.305) (end 165.735 154.305) (width 0.4) (layer F.Cu) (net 34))
 (segment (start 165.735 154.305) (end 165.1 154.94) (width 0.4) (layer F.Cu) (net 34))
 (segment (start 169.29 155.575) (end 167.005 155.575) (width 0.4) (layer F.Cu) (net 35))
 (segment (start 167.005 155.575) (end 165.1 157.48) (width 0.4) (layer F.Cu) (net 35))
 (segment (start 165.1 160.02) (end 165.1 159.766) (width 0.4) (layer F.Cu) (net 36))
 (segment (start 165.1 159.766) (end 168.021 156.845) (width 0.4) (layer F.Cu) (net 36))
 (segment (start 168.021 156.845) (end 169.29 156.845) (width 0.4) (layer F.Cu) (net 36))
 (segment (start 169.29 158.115) (end 168.021 158.115) (width 0.4) (layer F.Cu) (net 37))
 (segment (start 167.132 160.528) (end 165.1 162.56) (width 0.4) (layer F.Cu) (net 37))
 (segment (start 167.132 159.004) (end 167.132 160.528) (width 0.4) (layer F.Cu) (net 37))
 (segment (start 168.021 158.115) (end 167.132 159.004) (width 0.4) (layer F.Cu) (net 37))
 (segment (start 165.1 165.1) (end 167.64 165.1) (width 0.4) (layer F.Cu) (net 38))
 (segment (start 169.29 163.45) (end 169.29 159.385) (width 0.4) (layer F.Cu) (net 38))
 (segment (start 167.64 165.1) (end 169.29 163.45) (width 0.4) (layer F.Cu) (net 38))
 (segment (start 182.88 165.1) (end 180.34 165.1) (width 0.4) (layer F.Cu) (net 48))
 (segment (start 178.69 163.45) (end 178.69 159.385) (width 0.4) (layer F.Cu) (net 48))
 (segment (start 180.34 165.1) (end 178.69 163.45) (width 0.4) (layer F.Cu) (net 48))
 (segment (start 178.69 158.115) (end 179.705 158.115) (width 0.4) (layer F.Cu) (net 47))
 (segment (start 180.594 160.274) (end 182.88 162.56) (width 0.4) (layer F.Cu) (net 47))
 (segment (start 180.594 159.004) (end 180.594 160.274) (width 0.4) (layer F.Cu) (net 47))
 (segment (start 179.705 158.115) (end 180.594 159.004) (width 0.4) (layer F.Cu) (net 47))
 (segment (start 178.69 156.845) (end 179.705 156.845) (width 0.4) (layer F.Cu) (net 46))
 (segment (start 179.705 156.845) (end 182.88 160.02) (width 0.4) (layer F.Cu) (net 46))
 (segment (start 178.69 155.575) (end 180.975 155.575) (width 0.4) (layer F.Cu) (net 45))
 (segment (start 180.975 155.575) (end 182.88 157.48) (width 0.4) (layer F.Cu) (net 45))
 (segment (start 178.69 154.305) (end 182.245 154.305) (width 0.4) (layer F.Cu) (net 44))
 (segment (start 182.245 154.305) (end 182.88 154.94) (width 0.4) (layer F.Cu) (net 44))
 (segment (start 178.69 153.035) (end 182.245 153.035) (width 0.4) (layer F.Cu) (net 43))
 (segment (start 182.245 153.035) (end 182.88 152.4) (width 0.4) (layer F.Cu) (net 43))
 (segment (start 178.69 151.765) (end 180.975 151.765) (width 0.4) (layer F.Cu) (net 42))
 (segment (start 180.975 151.765) (end 182.88 149.86) (width 0.4) (layer F.Cu) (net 42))
 (segment (start 182.88 147.32) (end 182.88 147.828) (width 0.4) (layer F.Cu) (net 41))
 (segment (start 182.88 147.828) (end 180.213 150.495) (width 0.4) (layer F.Cu) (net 41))
 (segment (start 180.213 150.495) (end 178.69 150.495) (width 0.4) (layer F.Cu) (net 41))
 (segment (start 178.69 149.225) (end 179.959 149.225) (width 0.4) (layer F.Cu) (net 40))
 (segment (start 180.848 146.812) (end 182.88 144.78) (width 0.4) (layer F.Cu) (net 40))
 (segment (start 180.848 148.336) (end 180.848 146.812) (width 0.4) (layer F.Cu) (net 40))
 (segment (start 179.959 149.225) (end 180.848 148.336) (width 0.4) (layer F.Cu) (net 40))
 (segment (start 178.69 147.955) (end 178.69 143.636) (width 0.4) (layer F.Cu) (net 39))
 (segment (start 180.086 142.24) (end 182.88 142.24) (width 0.4) (layer F.Cu) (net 39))
 (segment (start 178.69 143.636) (end 180.086 142.24) (width 0.4) (layer F.Cu) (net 39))
 (segment (start 182.88 104.14) (end 180.594 104.14) (width 0.4) (layer F.Cu) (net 14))
 (segment (start 177.8 111.505) (end 178.69 112.395) (width 0.4) (layer F.Cu) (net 14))
 (segment (start 177.8 106.934) (end 177.8 111.505) (width 0.4) (layer F.Cu) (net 14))
 (segment (start 180.594 104.14) (end 177.8 106.934) (width 0.4) (layer F.Cu) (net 14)))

